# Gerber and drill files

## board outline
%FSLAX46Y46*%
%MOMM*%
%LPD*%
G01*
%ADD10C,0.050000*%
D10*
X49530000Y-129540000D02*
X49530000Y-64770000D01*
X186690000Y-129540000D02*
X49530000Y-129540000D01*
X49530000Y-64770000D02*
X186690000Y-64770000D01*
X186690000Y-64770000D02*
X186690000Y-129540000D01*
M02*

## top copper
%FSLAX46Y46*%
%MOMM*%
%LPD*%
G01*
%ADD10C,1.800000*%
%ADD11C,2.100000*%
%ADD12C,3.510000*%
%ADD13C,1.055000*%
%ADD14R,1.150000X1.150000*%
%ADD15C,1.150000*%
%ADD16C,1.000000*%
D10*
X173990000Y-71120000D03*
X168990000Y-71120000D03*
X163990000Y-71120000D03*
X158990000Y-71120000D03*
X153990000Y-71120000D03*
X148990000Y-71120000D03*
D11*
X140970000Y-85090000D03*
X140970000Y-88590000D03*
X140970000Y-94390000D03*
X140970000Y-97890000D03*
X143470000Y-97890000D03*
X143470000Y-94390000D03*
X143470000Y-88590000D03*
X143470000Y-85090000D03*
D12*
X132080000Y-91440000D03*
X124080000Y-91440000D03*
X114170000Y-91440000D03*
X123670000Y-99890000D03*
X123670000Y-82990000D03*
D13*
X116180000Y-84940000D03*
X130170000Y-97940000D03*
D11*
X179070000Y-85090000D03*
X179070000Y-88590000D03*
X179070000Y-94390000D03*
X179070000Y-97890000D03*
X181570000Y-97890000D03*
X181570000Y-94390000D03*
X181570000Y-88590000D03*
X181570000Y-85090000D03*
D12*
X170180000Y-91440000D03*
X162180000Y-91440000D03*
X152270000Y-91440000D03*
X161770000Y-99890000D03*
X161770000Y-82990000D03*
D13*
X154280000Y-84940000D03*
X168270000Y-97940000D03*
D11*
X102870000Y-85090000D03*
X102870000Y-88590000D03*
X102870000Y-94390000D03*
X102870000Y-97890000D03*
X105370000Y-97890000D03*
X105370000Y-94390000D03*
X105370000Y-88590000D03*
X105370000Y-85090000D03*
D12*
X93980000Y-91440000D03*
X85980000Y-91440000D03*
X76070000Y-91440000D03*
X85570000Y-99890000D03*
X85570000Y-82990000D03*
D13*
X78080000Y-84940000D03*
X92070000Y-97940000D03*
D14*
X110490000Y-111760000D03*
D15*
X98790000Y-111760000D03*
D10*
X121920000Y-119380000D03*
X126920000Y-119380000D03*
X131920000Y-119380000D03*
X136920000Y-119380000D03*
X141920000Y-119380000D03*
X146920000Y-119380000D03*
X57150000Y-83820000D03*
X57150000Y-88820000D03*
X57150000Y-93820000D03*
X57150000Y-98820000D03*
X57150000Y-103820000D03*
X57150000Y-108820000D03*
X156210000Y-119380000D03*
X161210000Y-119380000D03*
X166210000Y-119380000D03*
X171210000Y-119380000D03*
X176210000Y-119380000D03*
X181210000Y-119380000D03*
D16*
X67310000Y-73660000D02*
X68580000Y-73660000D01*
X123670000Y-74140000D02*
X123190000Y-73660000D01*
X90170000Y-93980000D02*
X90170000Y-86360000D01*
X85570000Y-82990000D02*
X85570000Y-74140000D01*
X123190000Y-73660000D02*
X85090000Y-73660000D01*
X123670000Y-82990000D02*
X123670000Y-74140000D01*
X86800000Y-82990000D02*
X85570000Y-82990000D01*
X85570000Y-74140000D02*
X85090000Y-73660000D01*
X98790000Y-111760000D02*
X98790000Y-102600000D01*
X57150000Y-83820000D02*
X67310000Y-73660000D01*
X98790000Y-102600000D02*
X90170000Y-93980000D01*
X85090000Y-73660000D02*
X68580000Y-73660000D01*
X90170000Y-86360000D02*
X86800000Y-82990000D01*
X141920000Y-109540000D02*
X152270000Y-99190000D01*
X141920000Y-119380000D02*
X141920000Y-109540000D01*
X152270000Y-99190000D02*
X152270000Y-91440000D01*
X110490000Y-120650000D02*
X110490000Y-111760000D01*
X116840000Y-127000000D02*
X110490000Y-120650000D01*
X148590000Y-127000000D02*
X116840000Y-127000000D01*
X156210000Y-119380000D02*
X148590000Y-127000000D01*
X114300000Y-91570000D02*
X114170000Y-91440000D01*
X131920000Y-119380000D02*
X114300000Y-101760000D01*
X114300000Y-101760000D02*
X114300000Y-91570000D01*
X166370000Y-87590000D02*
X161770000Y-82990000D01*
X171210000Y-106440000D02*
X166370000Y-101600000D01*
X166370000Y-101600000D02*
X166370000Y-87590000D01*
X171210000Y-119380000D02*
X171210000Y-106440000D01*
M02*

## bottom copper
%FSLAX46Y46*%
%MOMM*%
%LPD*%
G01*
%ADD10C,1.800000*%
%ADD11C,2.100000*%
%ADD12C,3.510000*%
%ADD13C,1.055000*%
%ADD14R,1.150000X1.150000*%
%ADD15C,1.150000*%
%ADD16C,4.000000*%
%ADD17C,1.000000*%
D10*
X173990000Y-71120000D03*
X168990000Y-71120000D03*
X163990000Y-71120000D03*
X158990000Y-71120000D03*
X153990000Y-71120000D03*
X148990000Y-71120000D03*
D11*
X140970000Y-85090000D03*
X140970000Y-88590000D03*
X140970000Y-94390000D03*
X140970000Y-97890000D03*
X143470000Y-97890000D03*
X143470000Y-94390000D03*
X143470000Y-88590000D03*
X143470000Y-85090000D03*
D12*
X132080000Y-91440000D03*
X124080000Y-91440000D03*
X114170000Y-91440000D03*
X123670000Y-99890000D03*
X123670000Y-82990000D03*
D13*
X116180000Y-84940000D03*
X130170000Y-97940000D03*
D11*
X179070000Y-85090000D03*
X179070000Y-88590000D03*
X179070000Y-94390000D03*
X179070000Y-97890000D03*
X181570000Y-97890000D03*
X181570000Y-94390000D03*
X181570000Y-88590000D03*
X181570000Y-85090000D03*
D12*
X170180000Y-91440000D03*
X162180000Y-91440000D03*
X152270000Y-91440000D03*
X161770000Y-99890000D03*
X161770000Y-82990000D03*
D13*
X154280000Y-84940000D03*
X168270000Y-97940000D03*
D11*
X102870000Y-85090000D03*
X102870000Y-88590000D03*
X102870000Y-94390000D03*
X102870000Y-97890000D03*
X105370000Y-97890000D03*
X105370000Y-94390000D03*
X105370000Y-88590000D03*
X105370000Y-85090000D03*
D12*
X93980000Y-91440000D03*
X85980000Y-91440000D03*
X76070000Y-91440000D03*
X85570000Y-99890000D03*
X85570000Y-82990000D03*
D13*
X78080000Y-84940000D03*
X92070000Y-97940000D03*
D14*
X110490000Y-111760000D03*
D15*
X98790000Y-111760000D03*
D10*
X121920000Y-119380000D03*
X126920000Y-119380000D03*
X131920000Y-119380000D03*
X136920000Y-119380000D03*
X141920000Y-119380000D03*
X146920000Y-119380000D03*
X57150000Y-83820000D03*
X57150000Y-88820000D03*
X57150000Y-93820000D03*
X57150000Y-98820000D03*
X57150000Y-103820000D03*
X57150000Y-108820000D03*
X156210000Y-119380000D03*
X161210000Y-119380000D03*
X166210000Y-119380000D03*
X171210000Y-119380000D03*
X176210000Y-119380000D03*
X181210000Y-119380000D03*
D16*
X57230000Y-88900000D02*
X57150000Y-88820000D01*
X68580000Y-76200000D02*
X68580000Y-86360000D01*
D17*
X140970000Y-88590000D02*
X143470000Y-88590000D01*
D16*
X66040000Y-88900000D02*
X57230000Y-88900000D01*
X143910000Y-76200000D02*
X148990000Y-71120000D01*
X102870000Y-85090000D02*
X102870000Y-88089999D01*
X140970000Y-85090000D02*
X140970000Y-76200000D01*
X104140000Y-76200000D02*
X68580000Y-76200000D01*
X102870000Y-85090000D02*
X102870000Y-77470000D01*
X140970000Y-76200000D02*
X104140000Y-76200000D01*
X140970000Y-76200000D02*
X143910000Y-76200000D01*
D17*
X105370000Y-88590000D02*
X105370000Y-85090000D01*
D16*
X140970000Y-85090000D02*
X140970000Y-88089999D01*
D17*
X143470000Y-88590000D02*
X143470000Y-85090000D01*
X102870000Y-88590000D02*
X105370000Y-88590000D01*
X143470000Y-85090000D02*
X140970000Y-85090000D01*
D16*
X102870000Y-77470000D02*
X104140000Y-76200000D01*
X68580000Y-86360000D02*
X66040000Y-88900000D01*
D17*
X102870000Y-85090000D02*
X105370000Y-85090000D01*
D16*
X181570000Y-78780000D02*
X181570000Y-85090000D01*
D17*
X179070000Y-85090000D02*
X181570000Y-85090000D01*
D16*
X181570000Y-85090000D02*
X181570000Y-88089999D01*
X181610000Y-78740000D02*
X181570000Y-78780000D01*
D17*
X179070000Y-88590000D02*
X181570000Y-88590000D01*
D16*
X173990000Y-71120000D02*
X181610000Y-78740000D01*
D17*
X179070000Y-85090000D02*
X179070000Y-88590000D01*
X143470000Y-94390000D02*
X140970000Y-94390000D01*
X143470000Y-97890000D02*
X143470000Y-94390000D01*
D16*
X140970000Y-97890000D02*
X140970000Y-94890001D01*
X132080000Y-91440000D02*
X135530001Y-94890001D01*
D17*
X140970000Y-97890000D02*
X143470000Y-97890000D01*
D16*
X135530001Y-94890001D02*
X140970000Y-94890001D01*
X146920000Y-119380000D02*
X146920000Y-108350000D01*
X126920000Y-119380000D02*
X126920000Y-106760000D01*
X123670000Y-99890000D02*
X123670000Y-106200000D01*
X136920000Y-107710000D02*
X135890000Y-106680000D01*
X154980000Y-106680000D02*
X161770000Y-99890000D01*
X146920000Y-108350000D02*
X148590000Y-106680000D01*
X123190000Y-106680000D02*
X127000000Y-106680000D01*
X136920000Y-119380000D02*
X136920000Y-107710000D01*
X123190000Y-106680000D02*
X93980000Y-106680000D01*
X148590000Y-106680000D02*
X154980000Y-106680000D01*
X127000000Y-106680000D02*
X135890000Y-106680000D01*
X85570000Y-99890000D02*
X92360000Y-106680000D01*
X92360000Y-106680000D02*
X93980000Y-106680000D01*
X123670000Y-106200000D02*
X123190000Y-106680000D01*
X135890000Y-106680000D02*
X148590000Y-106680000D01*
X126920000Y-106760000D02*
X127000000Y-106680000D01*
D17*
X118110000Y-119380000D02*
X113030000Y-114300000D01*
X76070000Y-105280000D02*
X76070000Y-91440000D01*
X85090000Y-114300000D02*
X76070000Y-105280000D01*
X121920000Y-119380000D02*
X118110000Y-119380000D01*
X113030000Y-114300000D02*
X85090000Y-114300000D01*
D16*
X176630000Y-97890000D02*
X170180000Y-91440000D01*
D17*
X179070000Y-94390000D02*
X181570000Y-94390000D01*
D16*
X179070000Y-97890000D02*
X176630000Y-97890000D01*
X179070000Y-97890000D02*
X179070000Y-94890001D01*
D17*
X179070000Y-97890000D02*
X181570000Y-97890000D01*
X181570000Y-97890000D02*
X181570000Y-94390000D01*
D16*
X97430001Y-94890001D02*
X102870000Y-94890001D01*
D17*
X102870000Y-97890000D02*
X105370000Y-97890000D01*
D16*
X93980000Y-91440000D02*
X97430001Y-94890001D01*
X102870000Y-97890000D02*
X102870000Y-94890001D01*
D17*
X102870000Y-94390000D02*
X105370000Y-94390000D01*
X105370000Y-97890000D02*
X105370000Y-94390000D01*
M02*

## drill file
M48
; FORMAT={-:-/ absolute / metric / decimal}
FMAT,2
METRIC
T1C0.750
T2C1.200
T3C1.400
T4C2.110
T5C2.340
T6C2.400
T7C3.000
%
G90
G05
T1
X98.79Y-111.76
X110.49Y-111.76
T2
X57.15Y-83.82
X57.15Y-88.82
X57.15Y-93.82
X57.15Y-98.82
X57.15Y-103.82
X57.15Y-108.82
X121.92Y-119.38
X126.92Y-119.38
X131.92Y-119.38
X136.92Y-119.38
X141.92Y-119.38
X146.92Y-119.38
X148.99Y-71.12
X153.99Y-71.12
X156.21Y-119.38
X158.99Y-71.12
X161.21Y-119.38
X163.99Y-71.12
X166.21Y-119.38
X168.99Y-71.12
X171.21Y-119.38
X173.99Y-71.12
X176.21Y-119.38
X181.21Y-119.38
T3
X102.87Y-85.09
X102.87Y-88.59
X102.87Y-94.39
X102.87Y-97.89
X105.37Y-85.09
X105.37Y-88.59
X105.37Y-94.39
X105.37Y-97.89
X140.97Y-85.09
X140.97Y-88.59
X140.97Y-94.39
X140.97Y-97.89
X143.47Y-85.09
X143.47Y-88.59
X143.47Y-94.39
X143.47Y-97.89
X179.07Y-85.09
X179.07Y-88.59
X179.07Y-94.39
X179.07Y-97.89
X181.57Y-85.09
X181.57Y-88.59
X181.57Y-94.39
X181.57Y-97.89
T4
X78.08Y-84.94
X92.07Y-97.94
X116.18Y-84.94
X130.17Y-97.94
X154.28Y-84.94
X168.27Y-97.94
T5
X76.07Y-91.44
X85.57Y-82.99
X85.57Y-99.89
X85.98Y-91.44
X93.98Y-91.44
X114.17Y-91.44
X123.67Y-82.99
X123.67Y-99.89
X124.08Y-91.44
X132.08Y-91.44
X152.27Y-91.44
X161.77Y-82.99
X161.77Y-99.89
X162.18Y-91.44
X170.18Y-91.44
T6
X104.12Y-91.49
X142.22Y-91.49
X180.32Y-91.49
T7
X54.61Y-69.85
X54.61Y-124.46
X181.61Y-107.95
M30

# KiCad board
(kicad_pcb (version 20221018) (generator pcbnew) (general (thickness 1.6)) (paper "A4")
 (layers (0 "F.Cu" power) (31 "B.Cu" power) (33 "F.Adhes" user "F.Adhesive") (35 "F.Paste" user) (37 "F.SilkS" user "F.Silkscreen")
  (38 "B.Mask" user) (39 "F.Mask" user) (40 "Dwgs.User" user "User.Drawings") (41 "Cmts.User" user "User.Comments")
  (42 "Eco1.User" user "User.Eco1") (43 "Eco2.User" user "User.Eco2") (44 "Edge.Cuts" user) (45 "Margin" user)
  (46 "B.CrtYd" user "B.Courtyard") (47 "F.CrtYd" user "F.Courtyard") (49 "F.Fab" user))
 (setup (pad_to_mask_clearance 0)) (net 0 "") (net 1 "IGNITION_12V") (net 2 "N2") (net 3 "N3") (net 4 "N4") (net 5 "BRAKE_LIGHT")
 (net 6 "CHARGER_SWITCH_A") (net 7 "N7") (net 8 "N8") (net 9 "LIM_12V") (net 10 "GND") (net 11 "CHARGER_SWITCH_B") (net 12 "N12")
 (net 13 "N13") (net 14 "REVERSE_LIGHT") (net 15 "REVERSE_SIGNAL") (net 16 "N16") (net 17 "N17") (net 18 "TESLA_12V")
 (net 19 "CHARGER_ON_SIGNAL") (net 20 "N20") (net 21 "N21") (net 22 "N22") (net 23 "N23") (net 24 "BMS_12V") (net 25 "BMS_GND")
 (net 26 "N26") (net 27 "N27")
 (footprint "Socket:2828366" (layer "F.Cu") (at 173.99 71.12 180)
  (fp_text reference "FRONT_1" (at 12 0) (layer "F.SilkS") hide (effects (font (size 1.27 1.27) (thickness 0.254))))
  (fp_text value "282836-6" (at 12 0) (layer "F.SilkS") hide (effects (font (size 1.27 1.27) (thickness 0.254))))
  (pad "1" thru_hole circle (at 0 0 180) (size 1.8 1.8) (drill 1.2) (layers "*.Cu" "*.Mask") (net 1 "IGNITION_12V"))
  (pad "2" thru_hole circle (at 5 0 180) (size 1.8 1.8) (drill 1.2) (layers "*.Cu" "*.Mask") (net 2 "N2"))
  (pad "3" thru_hole circle (at 10 0 180) (size 1.8 1.8) (drill 1.2) (layers "*.Cu" "*.Mask") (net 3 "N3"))
  (pad "4" thru_hole circle (at 15 0 180) (size 1.8 1.8) (drill 1.2) (layers "*.Cu" "*.Mask") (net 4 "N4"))
  (pad "5" thru_hole circle (at 20 0 180) (size 1.8 1.8) (drill 1.2) (layers "*.Cu" "*.Mask") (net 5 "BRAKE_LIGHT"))
  (pad "6" thru_hole circle (at 25 0 180) (size 1.8 1.8) (drill 1.2) (layers "*.Cu" "*.Mask") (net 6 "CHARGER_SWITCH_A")))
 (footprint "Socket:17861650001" (layer "F.Cu") (at 140.97 85.09 -90)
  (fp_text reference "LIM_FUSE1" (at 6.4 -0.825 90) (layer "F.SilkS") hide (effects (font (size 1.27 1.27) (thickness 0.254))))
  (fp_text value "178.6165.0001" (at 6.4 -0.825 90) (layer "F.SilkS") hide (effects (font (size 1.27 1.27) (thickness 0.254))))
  (pad "" np_thru_hole circle (at 6.4 -1.25 270) (size 0.001 0.001) (drill 2.4) (layers "*.Cu" "*.Mask"))
  (pad "1" thru_hole circle (at 0 0 270) (size 2.1 2.1) (drill 1.4) (layers "*.Cu" "*.Mask") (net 6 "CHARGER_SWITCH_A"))
  (pad "2" thru_hole circle (at 3.5 0 270) (size 2.1 2.1) (drill 1.4) (layers "*.Cu" "*.Mask") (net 6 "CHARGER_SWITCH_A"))
  (pad "3" thru_hole circle (at 9.3 0 270) (size 2.1 2.1) (drill 1.4) (layers "*.Cu" "*.Mask") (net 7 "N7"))
  (pad "4" thru_hole circle (at 12.8 0 270) (size 2.1 2.1) (drill 1.4) (layers "*.Cu" "*.Mask") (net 7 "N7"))
  (pad "5" thru_hole circle (at 12.8 -2.5 270) (size 2.1 2.1) (drill 1.4) (layers "*.Cu" "*.Mask") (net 7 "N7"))
  (pad "6" thru_hole circle (at 9.3 -2.5 270) (size 2.1 2.1) (drill 1.4) (layers "*.Cu" "*.Mask") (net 7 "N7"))
  (pad "7" thru_hole circle (at 3.5 -2.5 270) (size 2.1 2.1) (drill 1.4) (layers "*.Cu" "*.Mask") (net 6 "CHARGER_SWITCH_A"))
  (pad "8" thru_hole circle (at 0 -2.5 270) (size 2.1 2.1) (drill 1.4) (layers "*.Cu" "*.Mask") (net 6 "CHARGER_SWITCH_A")))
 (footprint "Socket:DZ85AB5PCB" (layer "F.Cu") (at 132.08 91.44 180)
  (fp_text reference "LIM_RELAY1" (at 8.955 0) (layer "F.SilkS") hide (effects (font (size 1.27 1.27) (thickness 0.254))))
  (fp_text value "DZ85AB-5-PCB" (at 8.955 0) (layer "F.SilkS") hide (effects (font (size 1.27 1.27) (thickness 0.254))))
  (pad "1" thru_hole circle (at 0 0 270) (size 3.51 3.51) (drill 2.34) (layers "*.Cu" "*.Mask" "F.SilkS") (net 7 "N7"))
  (pad "2" thru_hole circle (at 8 0 270) (size 3.51 3.51) (drill 2.34) (layers "*.Cu" "*.Mask" "F.SilkS") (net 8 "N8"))
  (pad "3" thru_hole circle (at 17.91 0 270) (size 3.51 3.51) (drill 2.34) (layers "*.Cu" "*.Mask" "F.SilkS") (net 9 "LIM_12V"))
  (pad "4" thru_hole circle (at 8.41 -8.45 270) (size 3.51 3.51) (drill 2.34) (layers "*.Cu" "*.Mask" "F.SilkS") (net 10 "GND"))
  (pad "5" thru_hole circle (at 8.41 8.45 270) (size 3.51 3.51) (drill 2.34) (layers "*.Cu" "*.Mask" "F.SilkS") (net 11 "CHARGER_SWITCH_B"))
  (pad "MH1" thru_hole circle (at 15.9 6.5 270) (size 1.055 1.055) (drill 2.11) (layers "*.Cu" "*.Mask" "F.SilkS"))
  (pad "MH2" thru_hole circle (at 1.91 -6.5 270) (size 1.055 1.055) (drill 2.11) (layers "*.Cu" "*.Mask" "F.SilkS")))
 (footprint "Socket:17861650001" (layer "F.Cu") (at 179.07 85.09 -90)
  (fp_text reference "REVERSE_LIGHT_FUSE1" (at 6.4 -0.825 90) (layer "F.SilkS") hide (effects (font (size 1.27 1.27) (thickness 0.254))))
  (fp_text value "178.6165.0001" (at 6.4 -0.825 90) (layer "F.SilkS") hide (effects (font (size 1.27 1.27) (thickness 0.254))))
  (pad "" np_thru_hole circle (at 6.4 -1.25 270) (size 0.001 0.001) (drill 2.4) (layers "*.Cu" "*.Mask"))
  (pad "1" thru_hole circle (at 0 0 270) (size 2.1 2.1) (drill 1.4) (layers "*.Cu" "*.Mask") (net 1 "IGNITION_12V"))
  (pad "2" thru_hole circle (at 3.5 0 270) (size 2.1 2.1) (drill 1.4) (layers "*.Cu" "*.Mask") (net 1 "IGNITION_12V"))
  (pad "3" thru_hole circle (at 9.3 0 270) (size 2.1 2.1) (drill 1.4) (layers "*.Cu" "*.Mask") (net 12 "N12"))
  (pad "4" thru_hole circle (at 12.8 0 270) (size 2.1 2.1) (drill 1.4) (layers "*.Cu" "*.Mask") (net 12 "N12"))
  (pad "5" thru_hole circle (at 12.8 -2.5 270) (size 2.1 2.1) (drill 1.4) (layers "*.Cu" "*.Mask") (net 12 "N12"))
  (pad "6" thru_hole circle (at 9.3 -2.5 270) (size 2.1 2.1) (drill 1.4) (layers "*.Cu" "*.Mask") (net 12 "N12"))
  (pad "7" thru_hole circle (at 3.5 -2.5 270) (size 2.1 2.1) (drill 1.4) (layers "*.Cu" "*.Mask") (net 1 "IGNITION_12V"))
  (pad "8" thru_hole circle (at 0 -2.5 270) (size 2.1 2.1) (drill 1.4) (layers "*.Cu" "*.Mask") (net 1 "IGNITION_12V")))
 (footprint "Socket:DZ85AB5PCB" (layer "F.Cu") (at 170.18 91.44 180)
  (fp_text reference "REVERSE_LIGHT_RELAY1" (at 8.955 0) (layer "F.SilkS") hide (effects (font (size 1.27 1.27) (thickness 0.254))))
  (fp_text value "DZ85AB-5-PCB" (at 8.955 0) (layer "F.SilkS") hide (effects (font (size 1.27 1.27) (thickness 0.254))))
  (pad "1" thru_hole circle (at 0 0 270) (size 3.51 3.51) (drill 2.34) (layers "*.Cu" "*.Mask" "F.SilkS") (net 12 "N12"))
  (pad "2" thru_hole circle (at 8 0 270) (size 3.51 3.51) (drill 2.34) (layers "*.Cu" "*.Mask" "F.SilkS") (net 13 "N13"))
  (pad "3" thru_hole circle (at 17.91 0 270) (size 3.51 3.51) (drill 2.34) (layers "*.Cu" "*.Mask" "F.SilkS") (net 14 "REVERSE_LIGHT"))
  (pad "4" thru_hole circle (at 8.41 -8.45 270) (size 3.51 3.51) (drill 2.34) (layers "*.Cu" "*.Mask" "F.SilkS") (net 10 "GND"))
  (pad "5" thru_hole circle (at 8.41 8.45 270) (size 3.51 3.51) (drill 2.34) (layers "*.Cu" "*.Mask" "F.SilkS") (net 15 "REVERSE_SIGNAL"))
  (pad "MH1" thru_hole circle (at 15.9 6.5 270) (size 1.055 1.055) (drill 2.11) (layers "*.Cu" "*.Mask" "F.SilkS"))
  (pad "MH2" thru_hole circle (at 1.91 -6.5 270) (size 1.055 1.055) (drill 2.11) (layers "*.Cu" "*.Mask" "F.SilkS")))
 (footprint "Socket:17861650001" (layer "F.Cu") (at 102.87 85.09 -90)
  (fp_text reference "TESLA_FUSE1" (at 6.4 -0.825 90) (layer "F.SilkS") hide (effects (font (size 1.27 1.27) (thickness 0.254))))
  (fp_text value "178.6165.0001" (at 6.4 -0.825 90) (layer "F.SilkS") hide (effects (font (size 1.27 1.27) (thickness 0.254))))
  (pad "" np_thru_hole circle (at 6.4 -1.25 270) (size 0.001 0.001) (drill 2.4) (layers "*.Cu" "*.Mask"))
  (pad "1" thru_hole circle (at 0 0 270) (size 2.1 2.1) (drill 1.4) (layers "*.Cu" "*.Mask") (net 6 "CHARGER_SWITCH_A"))
  (pad "2" thru_hole circle (at 3.5 0 270) (size 2.1 2.1) (drill 1.4) (layers "*.Cu" "*.Mask") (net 6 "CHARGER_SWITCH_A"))
  (pad "3" thru_hole circle (at 9.3 0 270) (size 2.1 2.1) (drill 1.4) (layers "*.Cu" "*.Mask") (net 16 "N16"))
  (pad "4" thru_hole circle (at 12.8 0 270) (size 2.1 2.1) (drill 1.4) (layers "*.Cu" "*.Mask") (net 16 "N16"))
  (pad "5" thru_hole circle (at 12.8 -2.5 270) (size 2.1 2.1) (drill 1.4) (layers "*.Cu" "*.Mask") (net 16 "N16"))
  (pad "6" thru_hole circle (at 9.3 -2.5 270) (size 2.1 2.1) (drill 1.4) (layers "*.Cu" "*.Mask") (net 16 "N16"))
  (pad "7" thru_hole circle (at 3.5 -2.5 270) (size 2.1 2.1) (drill 1.4) (layers "*.Cu" "*.Mask") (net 6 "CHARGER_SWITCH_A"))
  (pad "8" thru_hole circle (at 0 -2.5 270) (size 2.1 2.1) (drill 1.4) (layers "*.Cu" "*.Mask") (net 6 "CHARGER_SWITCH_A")))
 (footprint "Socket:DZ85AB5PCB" (layer "F.Cu") (at 93.98 91.44 180)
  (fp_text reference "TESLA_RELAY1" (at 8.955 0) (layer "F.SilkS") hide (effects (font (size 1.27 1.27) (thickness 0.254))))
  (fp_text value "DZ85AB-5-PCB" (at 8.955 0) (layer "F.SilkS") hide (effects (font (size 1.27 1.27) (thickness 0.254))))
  (pad "1" thru_hole circle (at 0 0 270) (size 3.51 3.51) (drill 2.34) (layers "*.Cu" "*.Mask" "F.SilkS") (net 16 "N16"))
  (pad "2" thru_hole circle (at 8 0 270) (size 3.51 3.51) (drill 2.34) (layers "*.Cu" "*.Mask" "F.SilkS") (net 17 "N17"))
  (pad "3" thru_hole circle (at 17.91 0 270) (size 3.51 3.51) (drill 2.34) (layers "*.Cu" "*.Mask" "F.SilkS") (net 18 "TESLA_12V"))
  (pad "4" thru_hole circle (at 8.41 -8.45 270) (size 3.51 3.51) (drill 2.34) (layers "*.Cu" "*.Mask" "F.SilkS") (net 10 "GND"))
  (pad "5" thru_hole circle (at 8.41 8.45 270) (size 3.51 3.51) (drill 2.34) (layers "*.Cu" "*.Mask" "F.SilkS") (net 11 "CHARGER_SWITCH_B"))
  (pad "MH1" thru_hole circle (at 15.9 6.5 270) (size 1.055 1.055) (drill 2.11) (layers "*.Cu" "*.Mask" "F.SilkS"))
  (pad "MH2" thru_hole circle (at 1.91 -6.5 270) (size 1.055 1.055) (drill 2.11) (layers "*.Cu" "*.Mask" "F.SilkS")))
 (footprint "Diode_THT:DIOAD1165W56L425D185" (layer "F.Cu") (at 110.49 111.76 180)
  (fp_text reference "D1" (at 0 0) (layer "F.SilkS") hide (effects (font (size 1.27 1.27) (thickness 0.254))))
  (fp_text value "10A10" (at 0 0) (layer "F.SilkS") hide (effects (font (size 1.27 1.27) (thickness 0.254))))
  (pad "1" thru_hole rect (at 0 0 180) (size 1.15 1.15) (drill 0.75) (layers "*.Cu" "*.Mask") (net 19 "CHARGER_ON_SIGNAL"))
  (pad "2" thru_hole circle (at 11.7 0 180) (size 1.15 1.15) (drill 0.75) (layers "*.Cu" "*.Mask") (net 11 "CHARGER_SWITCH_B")))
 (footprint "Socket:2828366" (layer "F.Cu") (at 121.92 119.38)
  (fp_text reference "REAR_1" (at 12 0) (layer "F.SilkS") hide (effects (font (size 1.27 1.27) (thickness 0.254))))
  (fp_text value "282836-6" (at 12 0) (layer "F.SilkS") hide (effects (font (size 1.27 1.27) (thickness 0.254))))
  (pad "1" thru_hole circle (at 0 0) (size 1.8 1.8) (drill 1.2) (layers "*.Cu" "*.Mask") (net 18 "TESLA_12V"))
  (pad "2" thru_hole circle (at 5 0) (size 1.8 1.8) (drill 1.2) (layers "*.Cu" "*.Mask") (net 10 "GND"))
  (pad "3" thru_hole circle (at 10 0) (size 1.8 1.8) (drill 1.2) (layers "*.Cu" "*.Mask") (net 9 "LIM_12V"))
  (pad "4" thru_hole circle (at 15 0) (size 1.8 1.8) (drill 1.2) (layers "*.Cu" "*.Mask") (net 10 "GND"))
  (pad "5" thru_hole circle (at 20 0) (size 1.8 1.8) (drill 1.2) (layers "*.Cu" "*.Mask") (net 14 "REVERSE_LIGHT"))
  (pad "6" thru_hole circle (at 25 0) (size 1.8 1.8) (drill 1.2) (layers "*.Cu" "*.Mask") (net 10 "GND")))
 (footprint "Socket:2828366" (layer "F.Cu") (at 57.15 83.82 -90)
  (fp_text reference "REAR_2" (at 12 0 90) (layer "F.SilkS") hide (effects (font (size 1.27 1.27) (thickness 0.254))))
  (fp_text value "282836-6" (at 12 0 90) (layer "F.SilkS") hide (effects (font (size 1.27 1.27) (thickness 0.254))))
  (pad "1" thru_hole circle (at 0 0 270) (size 1.8 1.8) (drill 1.2) (layers "*.Cu" "*.Mask") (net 11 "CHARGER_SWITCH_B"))
  (pad "2" thru_hole circle (at 5 0 270) (size 1.8 1.8) (drill 1.2) (layers "*.Cu" "*.Mask") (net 6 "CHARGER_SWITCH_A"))
  (pad "3" thru_hole circle (at 10 0 270) (size 1.8 1.8) (drill 1.2) (layers "*.Cu" "*.Mask") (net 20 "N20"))
  (pad "4" thru_hole circle (at 15 0 270) (size 1.8 1.8) (drill 1.2) (layers "*.Cu" "*.Mask") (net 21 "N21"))
  (pad "5" thru_hole circle (at 20 0 270) (size 1.8 1.8) (drill 1.2) (layers "*.Cu" "*.Mask") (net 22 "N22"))
  (pad "6" thru_hole circle (at 25 0 270) (size 1.8 1.8) (drill 1.2) (layers "*.Cu" "*.Mask") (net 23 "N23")))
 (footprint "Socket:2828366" (layer "F.Cu") (at 156.21 119.38)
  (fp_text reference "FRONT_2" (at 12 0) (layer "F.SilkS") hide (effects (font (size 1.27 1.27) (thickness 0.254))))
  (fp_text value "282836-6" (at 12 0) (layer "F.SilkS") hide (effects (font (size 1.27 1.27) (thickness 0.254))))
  (pad "1" thru_hole circle (at 0 0) (size 1.8 1.8) (drill 1.2) (layers "*.Cu" "*.Mask") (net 19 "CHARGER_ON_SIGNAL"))
  (pad "2" thru_hole circle (at 5 0) (size 1.8 1.8) (drill 1.2) (layers "*.Cu" "*.Mask") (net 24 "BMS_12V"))
  (pad "3" thru_hole circle (at 10 0) (size 1.8 1.8) (drill 1.2) (layers "*.Cu" "*.Mask") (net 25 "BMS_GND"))
  (pad "4" thru_hole circle (at 15 0) (size 1.8 1.8) (drill 1.2) (layers "*.Cu" "*.Mask") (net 15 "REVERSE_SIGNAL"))
  (pad "5" thru_hole circle (at 20 0) (size 1.8 1.8) (drill 1.2) (layers "*.Cu" "*.Mask") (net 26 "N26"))
  (pad "6" thru_hole circle (at 25 0) (size 1.8 1.8) (drill 1.2) (layers "*.Cu" "*.Mask") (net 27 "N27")))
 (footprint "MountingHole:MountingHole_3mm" (layer "F.Cu") (at 54.61 69.85)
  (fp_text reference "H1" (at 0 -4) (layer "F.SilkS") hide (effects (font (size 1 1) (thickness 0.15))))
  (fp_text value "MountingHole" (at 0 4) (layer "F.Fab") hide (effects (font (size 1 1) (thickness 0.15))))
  (pad "" np_thru_hole circle (at 0 0) (size 3 3) (drill 3) (layers "*.Cu" "*.Mask")))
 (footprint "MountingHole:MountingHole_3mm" (layer "F.Cu") (at 54.61 124.46)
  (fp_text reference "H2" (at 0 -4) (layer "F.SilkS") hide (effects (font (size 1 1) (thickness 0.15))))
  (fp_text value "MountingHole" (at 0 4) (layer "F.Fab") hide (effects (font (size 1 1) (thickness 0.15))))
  (pad "" np_thru_hole circle (at 0 0) (size 3 3) (drill 3) (layers "*.Cu" "*.Mask")))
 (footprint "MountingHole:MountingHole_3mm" (layer "F.Cu") (at 181.61 107.95)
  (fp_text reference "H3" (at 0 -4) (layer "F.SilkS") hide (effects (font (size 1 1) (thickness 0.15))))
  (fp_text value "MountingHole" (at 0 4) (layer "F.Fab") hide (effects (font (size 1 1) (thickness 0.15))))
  (pad "" np_thru_hole circle (at 0 0) (size 3 3) (drill 3) (layers "*.Cu" "*.Mask")))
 (gr_line (start 49.53 129.54) (end 49.53 64.77) (stroke (width 0.05) (type solid)) (layer "Edge.Cuts"))
 (gr_line (start 186.69 129.54) (end 49.53 129.54) (stroke (width 0.05) (type solid)) (layer "Edge.Cuts"))
 (gr_line (start 49.53 64.77) (end 186.69 64.77) (stroke (width 0.05) (type solid)) (layer "Edge.Cuts"))
 (gr_line (start 186.69 64.77) (end 186.69 129.54) (stroke (width 0.05) (type solid)) (layer "Edge.Cuts"))
 (segment (start 57.23 88.9) (end 57.15 88.82) (width 4) (layer "B.Cu") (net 6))
 (segment (start 68.58 76.2) (end 68.58 86.36) (width 4) (layer "B.Cu") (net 6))
 (segment (start 140.97 88.59) (end 143.47 88.59) (width 1) (layer "B.Cu") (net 6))
 (segment (start 66.04 88.9) (end 57.23 88.9) (width 4) (layer "B.Cu") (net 6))
 (segment (start 143.91 76.2) (end 148.99 71.12) (width 4) (layer "B.Cu") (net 6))
 (segment (start 102.87 85.09) (end 102.87 88.089999) (width 4) (layer "B.Cu") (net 6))
 (segment (start 140.97 85.09) (end 140.97 76.2) (width 4) (layer "B.Cu") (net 6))
 (segment (start 104.14 76.2) (end 68.58 76.2) (width 4) (layer "B.Cu") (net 6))
 (segment (start 102.87 85.09) (end 102.87 77.47) (width 4) (layer "B.Cu") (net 6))
 (segment (start 140.97 76.2) (end 104.14 76.2) (width 4) (layer "B.Cu") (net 6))
 (segment (start 140.97 76.2) (end 143.91 76.2) (width 4) (layer "B.Cu") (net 6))
 (segment (start 105.37 88.59) (end 105.37 85.09) (width 1) (layer "B.Cu") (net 6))
 (segment (start 140.97 85.09) (end 140.97 88.089999) (width 4) (layer "B.Cu") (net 6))
 (segment (start 143.47 88.59) (end 143.47 85.09) (width 1) (layer "B.Cu") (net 6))
 (segment (start 102.87 88.59) (end 105.37 88.59) (width 1) (layer "B.Cu") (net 6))
 (segment (start 143.47 85.09) (end 140.97 85.09) (width 1) (layer "B.Cu") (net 6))
 (segment (start 102.87 77.47) (end 104.14 76.2) (width 4) (layer "B.Cu") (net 6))
 (segment (start 68.58 86.36) (end 66.04 88.9) (width 4) (layer "B.Cu") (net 6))
 (segment (start 102.87 85.09) (end 105.37 85.09) (width 1) (layer "B.Cu") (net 6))
 (segment (start 181.57 78.78) (end 181.57 85.09) (width 4) (layer "B.Cu") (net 1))
 (segment (start 179.07 85.09) (end 181.57 85.09) (width 1) (layer "B.Cu") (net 1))
 (segment (start 181.57 85.09) (end 181.57 88.089999) (width 4) (layer "B.Cu") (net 1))
 (segment (start 181.61 78.74) (end 181.57 78.78) (width 4) (layer "B.Cu") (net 1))
 (segment (start 179.07 88.59) (end 181.57 88.59) (width 1) (layer "B.Cu") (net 1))
 (segment (start 173.99 71.12) (end 181.61 78.74) (width 4) (layer "B.Cu") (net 1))
 (segment (start 179.07 85.09) (end 179.07 88.59) (width 1) (layer "B.Cu") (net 1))
 (segment (start 67.31 73.66) (end 68.58 73.66) (width 1) (layer "F.Cu") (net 11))
 (segment (start 123.67 74.14) (end 123.19 73.66) (width 1) (layer "F.Cu") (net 11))
 (segment (start 90.17 93.98) (end 90.17 86.36) (width 1) (layer "F.Cu") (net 11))
 (segment (start 85.57 82.99) (end 85.57 74.14) (width 1) (layer "F.Cu") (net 11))
 (segment (start 123.19 73.66) (end 85.09 73.66) (width 1) (layer "F.Cu") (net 11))
 (segment (start 123.67 82.99) (end 123.67 74.14) (width 1) (layer "F.Cu") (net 11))
 (segment (start 86.8 82.99) (end 85.57 82.99) (width 1) (layer "F.Cu") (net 11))
 (segment (start 85.57 74.14) (end 85.09 73.66) (width 1) (layer "F.Cu") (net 11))
 (segment (start 98.79 111.76) (end 98.79 102.6) (width 1) (layer "F.Cu") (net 11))
 (segment (start 57.15 83.82) (end 67.31 73.66) (width 1) (layer "F.Cu") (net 11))
 (segment (start 98.79 102.6) (end 90.17 93.98) (width 1) (layer "F.Cu") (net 11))
 (segment (start 85.09 73.66) (end 68.58 73.66) (width 1) (layer "F.Cu") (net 11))
 (segment (start 90.17 86.36) (end 86.8 82.99) (width 1) (layer "F.Cu") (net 11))
 (segment (start 143.47 94.39) (end 140.97 94.39) (width 1) (layer "B.Cu") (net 7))
 (segment (start 143.47 97.89) (end 143.47 94.39) (width 1) (layer "B.Cu") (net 7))
 (segment (start 140.97 97.89) (end 140.97 94.890001) (width 4) (layer "B.Cu") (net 7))
 (segment (start 132.08 91.44) (end 135.530001 94.890001) (width 4) (layer "B.Cu") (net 7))
 (segment (start 140.97 97.89) (end 143.47 97.89) (width 1) (layer "B.Cu") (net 7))
 (segment (start 135.530001 94.890001) (end 140.97 94.890001) (width 4) (layer "B.Cu") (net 7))
 (segment (start 146.92 119.38) (end 146.92 108.35) (width 4) (layer "B.Cu") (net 10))
 (segment (start 126.92 119.38) (end 126.92 106.76) (width 4) (layer "B.Cu") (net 10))
 (segment (start 123.67 99.89) (end 123.67 106.2) (width 4) (layer "B.Cu") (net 10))
 (segment (start 136.92 107.71) (end 135.89 106.68) (width 4) (layer "B.Cu") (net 10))
 (segment (start 154.98 106.68) (end 161.77 99.89) (width 4) (layer "B.Cu") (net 10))
 (segment (start 146.92 108.35) (end 148.59 106.68) (width 4) (layer "B.Cu") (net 10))
 (segment (start 123.19 106.68) (end 127 106.68) (width 4) (layer "B.Cu") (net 10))
 (segment (start 136.92 119.38) (end 136.92 107.71) (width 4) (layer "B.Cu") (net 10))
 (segment (start 123.19 106.68) (end 93.98 106.68) (width 4) (layer "B.Cu") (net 10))
 (segment (start 148.59 106.68) (end 154.98 106.68) (width 4) (layer "B.Cu") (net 10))
 (segment (start 127 106.68) (end 135.89 106.68) (width 4) (layer "B.Cu") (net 10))
 (segment (start 85.57 99.89) (end 92.36 106.68) (width 4) (layer "B.Cu") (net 10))
 (segment (start 92.36 106.68) (end 93.98 106.68) (width 4) (layer "B.Cu") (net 10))
 (segment (start 123.67 106.2) (end 123.19 106.68) (width 4) (layer "B.Cu") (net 10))
 (segment (start 135.89 106.68) (end 148.59 106.68) (width 4) (layer "B.Cu") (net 10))
 (segment (start 126.92 106.76) (end 127 106.68) (width 4) (layer "B.Cu") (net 10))
 (segment (start 118.11 119.38) (end 113.03 114.3) (width 1) (layer "B.Cu") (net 18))
 (segment (start 76.07 105.28) (end 76.07 91.44) (width 1) (layer "B.Cu") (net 18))
 (segment (start 85.09 114.3) (end 76.07 105.28) (width 1) (layer "B.Cu") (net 18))
 (segment (start 121.92 119.38) (end 118.11 119.38) (width 1) (layer "B.Cu") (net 18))
 (segment (start 113.03 114.3) (end 85.09 114.3) (width 1) (layer "B.Cu") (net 18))
 (segment (start 176.63 97.89) (end 170.18 91.44) (width 4) (layer "B.Cu") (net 12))
 (segment (start 179.07 94.39) (end 181.57 94.39) (width 1) (layer "B.Cu") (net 12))
 (segment (start 179.07 97.89) (end 176.63 97.89) (width 4) (layer "B.Cu") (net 12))
 (segment (start 179.07 97.89) (end 179.07 94.890001) (width 4) (layer "B.Cu") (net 12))
 (segment (start 179.07 97.89) (end 181.57 97.89) (width 1) (layer "B.Cu") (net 12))
 (segment (start 181.57 97.89) (end 181.57 94.39) (width 1) (layer "B.Cu") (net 12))
 (segment (start 141.92 109.54) (end 152.27 99.19) (width 1) (layer "F.Cu") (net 14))
 (segment (start 141.92 119.38) (end 141.92 109.54) (width 1) (layer "F.Cu") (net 14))
 (segment (start 152.27 99.19) (end 152.27 91.44) (width 1) (layer "F.Cu") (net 14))
 (segment (start 97.430001 94.890001) (end 102.87 94.890001) (width 4) (layer "B.Cu") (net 16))
 (segment (start 102.87 97.89) (end 105.37 97.89) (width 1) (layer "B.Cu") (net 16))
 (segment (start 93.98 91.44) (end 97.430001 94.890001) (width 4) (layer "B.Cu") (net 16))
 (segment (start 102.87 97.89) (end 102.87 94.890001) (width 4) (layer "B.Cu") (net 16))
 (segment (start 102.87 94.39) (end 105.37 94.39) (width 1) (layer "B.Cu") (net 16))
 (segment (start 105.37 97.89) (end 105.37 94.39) (width 1) (layer "B.Cu") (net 16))
 (segment (start 110.49 120.65) (end 110.49 111.76) (width 1) (layer "F.Cu") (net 19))
 (segment (start 116.84 127) (end 110.49 120.65) (width 1) (layer "F.Cu") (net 19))
 (segment (start 148.59 127) (end 116.84 127) (width 1) (layer "F.Cu") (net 19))
 (segment (start 156.21 119.38) (end 148.59 127) (width 1) (layer "F.Cu") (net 19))
 (segment (start 114.3 91.57) (end 114.17 91.44) (width 1) (layer "F.Cu") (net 9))
 (segment (start 131.92 119.38) (end 114.3 101.76) (width 1) (layer "F.Cu") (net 9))
 (segment (start 114.3 101.76) (end 114.3 91.57) (width 1) (layer "F.Cu") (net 9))
 (segment (start 166.37 87.59) (end 161.77 82.99) (width 1) (layer "F.Cu") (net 15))
 (segment (start 171.21 106.44) (end 166.37 101.6) (width 1) (layer "F.Cu") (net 15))
 (segment (start 166.37 101.6) (end 166.37 87.59) (width 1) (layer "F.Cu") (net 15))
 (segment (start 171.21 119.38) (end 171.21 106.44) (width 1) (layer "F.Cu") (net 15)))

